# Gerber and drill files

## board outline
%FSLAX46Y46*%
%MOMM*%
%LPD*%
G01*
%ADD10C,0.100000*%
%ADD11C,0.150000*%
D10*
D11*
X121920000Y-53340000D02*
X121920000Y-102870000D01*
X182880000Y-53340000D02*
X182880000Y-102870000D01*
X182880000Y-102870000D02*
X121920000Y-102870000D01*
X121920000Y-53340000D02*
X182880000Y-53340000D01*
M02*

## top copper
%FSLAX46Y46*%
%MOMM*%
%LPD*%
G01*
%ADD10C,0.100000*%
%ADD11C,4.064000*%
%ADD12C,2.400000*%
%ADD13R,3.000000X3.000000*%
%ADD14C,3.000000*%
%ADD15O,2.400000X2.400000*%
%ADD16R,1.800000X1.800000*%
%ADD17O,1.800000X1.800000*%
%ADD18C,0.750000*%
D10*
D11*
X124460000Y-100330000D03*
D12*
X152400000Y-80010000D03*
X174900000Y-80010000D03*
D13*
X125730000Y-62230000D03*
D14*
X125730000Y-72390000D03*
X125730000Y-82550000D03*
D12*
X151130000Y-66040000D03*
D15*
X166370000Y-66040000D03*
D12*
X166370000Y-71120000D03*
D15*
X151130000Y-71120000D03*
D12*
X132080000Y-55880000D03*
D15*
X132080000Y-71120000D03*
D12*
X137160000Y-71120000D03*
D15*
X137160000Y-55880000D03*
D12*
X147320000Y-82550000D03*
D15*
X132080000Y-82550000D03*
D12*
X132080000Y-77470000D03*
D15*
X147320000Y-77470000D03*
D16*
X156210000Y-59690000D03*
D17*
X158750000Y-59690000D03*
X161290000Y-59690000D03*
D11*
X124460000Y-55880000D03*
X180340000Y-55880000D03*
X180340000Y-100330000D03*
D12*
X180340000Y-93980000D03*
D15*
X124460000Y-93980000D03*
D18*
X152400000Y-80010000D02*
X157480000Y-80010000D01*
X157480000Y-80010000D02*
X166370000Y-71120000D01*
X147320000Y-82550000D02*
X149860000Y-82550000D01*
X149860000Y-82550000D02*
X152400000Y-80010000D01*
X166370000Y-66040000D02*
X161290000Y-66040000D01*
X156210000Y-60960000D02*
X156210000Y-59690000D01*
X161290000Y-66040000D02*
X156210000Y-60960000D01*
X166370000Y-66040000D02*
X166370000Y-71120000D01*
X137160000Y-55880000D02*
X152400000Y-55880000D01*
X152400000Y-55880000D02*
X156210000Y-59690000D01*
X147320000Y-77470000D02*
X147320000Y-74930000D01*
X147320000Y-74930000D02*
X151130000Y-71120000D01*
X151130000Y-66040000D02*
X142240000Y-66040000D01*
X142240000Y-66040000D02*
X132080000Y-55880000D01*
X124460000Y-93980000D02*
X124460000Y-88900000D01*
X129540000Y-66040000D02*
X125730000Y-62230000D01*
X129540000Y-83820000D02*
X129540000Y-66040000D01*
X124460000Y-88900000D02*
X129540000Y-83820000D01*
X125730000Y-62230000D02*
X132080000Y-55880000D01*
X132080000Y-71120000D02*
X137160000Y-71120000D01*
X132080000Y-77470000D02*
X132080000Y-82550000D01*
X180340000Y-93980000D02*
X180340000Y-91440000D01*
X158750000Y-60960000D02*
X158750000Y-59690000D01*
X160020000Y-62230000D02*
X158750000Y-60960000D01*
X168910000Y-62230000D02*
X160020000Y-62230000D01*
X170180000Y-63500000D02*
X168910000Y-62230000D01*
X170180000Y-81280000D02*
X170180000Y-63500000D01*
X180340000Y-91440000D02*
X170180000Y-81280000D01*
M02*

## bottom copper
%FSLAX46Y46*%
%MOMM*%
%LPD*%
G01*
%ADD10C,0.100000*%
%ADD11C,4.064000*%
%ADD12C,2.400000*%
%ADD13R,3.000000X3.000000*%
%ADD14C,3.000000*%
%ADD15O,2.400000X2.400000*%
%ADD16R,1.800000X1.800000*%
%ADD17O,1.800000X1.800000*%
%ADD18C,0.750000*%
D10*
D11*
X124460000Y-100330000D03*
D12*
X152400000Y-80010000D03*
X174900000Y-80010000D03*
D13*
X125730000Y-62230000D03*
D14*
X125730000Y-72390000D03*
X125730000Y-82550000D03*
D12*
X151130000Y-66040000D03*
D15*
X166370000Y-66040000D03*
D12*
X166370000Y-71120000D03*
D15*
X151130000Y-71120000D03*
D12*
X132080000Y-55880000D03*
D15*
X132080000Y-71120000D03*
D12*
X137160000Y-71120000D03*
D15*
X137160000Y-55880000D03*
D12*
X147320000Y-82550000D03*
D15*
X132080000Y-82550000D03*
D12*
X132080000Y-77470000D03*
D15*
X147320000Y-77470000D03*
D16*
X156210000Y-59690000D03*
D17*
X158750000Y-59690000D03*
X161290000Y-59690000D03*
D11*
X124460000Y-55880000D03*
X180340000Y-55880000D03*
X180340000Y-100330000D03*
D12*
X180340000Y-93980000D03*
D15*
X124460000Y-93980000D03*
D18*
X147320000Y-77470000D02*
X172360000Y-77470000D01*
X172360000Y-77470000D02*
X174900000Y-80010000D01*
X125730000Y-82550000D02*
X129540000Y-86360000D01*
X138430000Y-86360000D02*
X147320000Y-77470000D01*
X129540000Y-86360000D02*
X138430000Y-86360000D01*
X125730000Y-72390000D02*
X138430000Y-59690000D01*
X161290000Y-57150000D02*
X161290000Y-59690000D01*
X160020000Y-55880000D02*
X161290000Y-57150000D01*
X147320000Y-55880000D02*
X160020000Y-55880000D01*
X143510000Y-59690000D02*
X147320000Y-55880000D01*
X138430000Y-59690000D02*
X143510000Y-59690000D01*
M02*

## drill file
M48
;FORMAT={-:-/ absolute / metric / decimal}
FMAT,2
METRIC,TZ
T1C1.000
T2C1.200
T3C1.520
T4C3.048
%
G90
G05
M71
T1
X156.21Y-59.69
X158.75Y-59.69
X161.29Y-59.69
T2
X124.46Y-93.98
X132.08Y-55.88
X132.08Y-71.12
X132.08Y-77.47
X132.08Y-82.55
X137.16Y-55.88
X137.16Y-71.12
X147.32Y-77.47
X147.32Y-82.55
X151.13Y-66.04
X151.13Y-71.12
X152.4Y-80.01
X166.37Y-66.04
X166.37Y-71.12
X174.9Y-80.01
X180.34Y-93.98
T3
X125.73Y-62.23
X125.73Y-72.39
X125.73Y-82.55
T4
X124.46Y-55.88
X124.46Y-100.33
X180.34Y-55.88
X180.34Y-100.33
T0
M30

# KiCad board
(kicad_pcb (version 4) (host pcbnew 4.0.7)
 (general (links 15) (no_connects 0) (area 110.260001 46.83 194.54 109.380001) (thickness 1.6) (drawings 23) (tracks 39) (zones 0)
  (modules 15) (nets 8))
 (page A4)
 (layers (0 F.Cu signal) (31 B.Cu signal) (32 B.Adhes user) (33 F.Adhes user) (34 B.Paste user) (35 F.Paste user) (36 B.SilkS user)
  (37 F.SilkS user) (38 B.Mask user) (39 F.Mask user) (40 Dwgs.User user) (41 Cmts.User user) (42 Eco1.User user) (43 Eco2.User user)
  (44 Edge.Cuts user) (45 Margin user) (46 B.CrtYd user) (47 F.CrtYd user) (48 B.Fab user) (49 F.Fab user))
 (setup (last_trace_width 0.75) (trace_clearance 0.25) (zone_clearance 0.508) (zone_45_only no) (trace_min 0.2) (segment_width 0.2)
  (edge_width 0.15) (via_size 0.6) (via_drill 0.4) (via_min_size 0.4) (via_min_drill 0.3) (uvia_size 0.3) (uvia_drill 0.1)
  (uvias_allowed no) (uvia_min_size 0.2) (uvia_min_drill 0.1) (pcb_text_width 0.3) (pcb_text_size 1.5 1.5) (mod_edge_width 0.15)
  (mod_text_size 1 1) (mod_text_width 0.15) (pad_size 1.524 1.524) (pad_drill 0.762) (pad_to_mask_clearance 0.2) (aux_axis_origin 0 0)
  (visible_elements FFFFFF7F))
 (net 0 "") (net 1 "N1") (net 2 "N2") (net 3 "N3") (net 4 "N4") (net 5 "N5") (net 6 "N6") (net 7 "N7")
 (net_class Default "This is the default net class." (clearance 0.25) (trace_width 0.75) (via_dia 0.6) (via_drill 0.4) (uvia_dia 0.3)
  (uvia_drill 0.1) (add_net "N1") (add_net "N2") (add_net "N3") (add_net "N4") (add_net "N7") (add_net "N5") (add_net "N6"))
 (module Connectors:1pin (layer F.Cu) (at 124.46 100.33)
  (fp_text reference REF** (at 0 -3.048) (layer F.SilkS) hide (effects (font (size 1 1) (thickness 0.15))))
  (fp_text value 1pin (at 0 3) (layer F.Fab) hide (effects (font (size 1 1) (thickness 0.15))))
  (pad 1 thru_hole circle (at 0 0) (size 4.064 4.064) (drill 3.048) (layers *.Cu *.Mask)))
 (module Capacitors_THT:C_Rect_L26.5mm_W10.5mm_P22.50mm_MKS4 (layer F.Cu) (at 152.4 80.01)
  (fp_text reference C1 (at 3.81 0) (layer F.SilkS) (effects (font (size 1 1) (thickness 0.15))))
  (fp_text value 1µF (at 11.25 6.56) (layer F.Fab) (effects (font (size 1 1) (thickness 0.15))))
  (pad 1 thru_hole circle (at 0 0) (size 2.4 2.4) (drill 1.2) (layers *.Cu *.Mask) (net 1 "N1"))
  (pad 2 thru_hole circle (at 22.5 0) (size 2.4 2.4) (drill 1.2) (layers *.Cu *.Mask) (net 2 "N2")))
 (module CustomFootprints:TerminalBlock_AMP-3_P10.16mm (layer F.Cu) (at 125.73 62.23 270)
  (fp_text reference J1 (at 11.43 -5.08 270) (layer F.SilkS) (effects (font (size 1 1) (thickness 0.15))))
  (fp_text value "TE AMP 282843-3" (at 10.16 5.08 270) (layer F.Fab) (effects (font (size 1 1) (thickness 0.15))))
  (pad 1 thru_hole rect (at 0 0 270) (size 3 3) (drill 1.52) (layers *.Cu *.Mask) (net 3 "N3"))
  (pad 2 thru_hole circle (at 10.16 0 270) (size 3 3) (drill 1.52) (layers *.Cu *.Mask) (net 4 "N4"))
  (pad 3 thru_hole circle (at 20.32 0 270) (size 3 3) (drill 1.52) (layers *.Cu *.Mask) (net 2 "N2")))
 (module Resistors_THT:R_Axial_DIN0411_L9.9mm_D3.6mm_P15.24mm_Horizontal (layer F.Cu) (at 151.13 66.04)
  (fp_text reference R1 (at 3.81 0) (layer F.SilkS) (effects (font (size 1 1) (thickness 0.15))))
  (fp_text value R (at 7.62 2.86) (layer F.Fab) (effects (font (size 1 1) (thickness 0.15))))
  (pad 1 thru_hole circle (at 0 0) (size 2.4 2.4) (drill 1.2) (layers *.Cu *.Mask) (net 3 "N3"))
  (pad 2 thru_hole oval (at 15.24 0) (size 2.4 2.4) (drill 1.2) (layers *.Cu *.Mask) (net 1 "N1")))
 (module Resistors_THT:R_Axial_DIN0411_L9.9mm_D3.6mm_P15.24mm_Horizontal (layer F.Cu) (at 166.37 71.12 180)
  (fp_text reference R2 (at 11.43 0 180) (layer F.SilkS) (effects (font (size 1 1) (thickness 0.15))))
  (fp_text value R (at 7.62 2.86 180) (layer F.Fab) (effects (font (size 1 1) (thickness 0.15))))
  (pad 1 thru_hole circle (at 0 0 180) (size 2.4 2.4) (drill 1.2) (layers *.Cu *.Mask) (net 1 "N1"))
  (pad 2 thru_hole oval (at 15.24 0 180) (size 2.4 2.4) (drill 1.2) (layers *.Cu *.Mask) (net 2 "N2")))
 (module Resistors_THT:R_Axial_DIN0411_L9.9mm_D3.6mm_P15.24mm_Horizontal (layer F.Cu) (at 132.08 55.88 270)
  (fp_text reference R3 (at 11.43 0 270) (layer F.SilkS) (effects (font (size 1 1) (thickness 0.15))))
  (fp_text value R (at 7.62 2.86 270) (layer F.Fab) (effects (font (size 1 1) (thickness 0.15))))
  (pad 1 thru_hole circle (at 0 0 270) (size 2.4 2.4) (drill 1.2) (layers *.Cu *.Mask) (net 3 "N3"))
  (pad 2 thru_hole oval (at 15.24 0 270) (size 2.4 2.4) (drill 1.2) (layers *.Cu *.Mask) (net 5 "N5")))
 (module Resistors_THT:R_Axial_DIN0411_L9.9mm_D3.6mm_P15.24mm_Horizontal (layer F.Cu) (at 137.16 71.12 90)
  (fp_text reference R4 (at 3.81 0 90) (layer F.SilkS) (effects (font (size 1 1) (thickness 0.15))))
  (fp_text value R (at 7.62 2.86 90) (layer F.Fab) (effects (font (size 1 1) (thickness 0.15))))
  (pad 1 thru_hole circle (at 0 0 90) (size 2.4 2.4) (drill 1.2) (layers *.Cu *.Mask) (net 5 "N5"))
  (pad 2 thru_hole oval (at 15.24 0 90) (size 2.4 2.4) (drill 1.2) (layers *.Cu *.Mask) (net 1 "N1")))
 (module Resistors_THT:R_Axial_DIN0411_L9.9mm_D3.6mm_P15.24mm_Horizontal (layer F.Cu) (at 147.32 82.55 180)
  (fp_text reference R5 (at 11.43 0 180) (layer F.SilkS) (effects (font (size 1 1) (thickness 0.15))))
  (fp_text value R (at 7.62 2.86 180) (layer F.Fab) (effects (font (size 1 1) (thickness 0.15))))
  (pad 1 thru_hole circle (at 0 0 180) (size 2.4 2.4) (drill 1.2) (layers *.Cu *.Mask) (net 1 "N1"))
  (pad 2 thru_hole oval (at 15.24 0 180) (size 2.4 2.4) (drill 1.2) (layers *.Cu *.Mask) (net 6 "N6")))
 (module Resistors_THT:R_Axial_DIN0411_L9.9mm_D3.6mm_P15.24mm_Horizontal (layer F.Cu) (at 132.08 77.47)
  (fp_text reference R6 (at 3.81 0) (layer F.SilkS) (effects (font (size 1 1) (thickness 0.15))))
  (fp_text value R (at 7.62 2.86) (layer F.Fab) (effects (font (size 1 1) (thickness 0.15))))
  (pad 1 thru_hole circle (at 0 0) (size 2.4 2.4) (drill 1.2) (layers *.Cu *.Mask) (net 6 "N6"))
  (pad 2 thru_hole oval (at 15.24 0) (size 2.4 2.4) (drill 1.2) (layers *.Cu *.Mask) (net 2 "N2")))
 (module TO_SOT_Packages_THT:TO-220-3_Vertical (layer F.Cu) (at 156.21 59.69)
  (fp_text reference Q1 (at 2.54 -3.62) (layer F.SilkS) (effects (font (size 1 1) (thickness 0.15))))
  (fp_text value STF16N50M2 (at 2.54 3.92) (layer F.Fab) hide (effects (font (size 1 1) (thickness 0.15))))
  (pad 1 thru_hole rect (at 0 0) (size 1.8 1.8) (drill 1) (layers *.Cu *.Mask) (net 1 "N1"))
  (pad 2 thru_hole oval (at 2.54 0) (size 1.8 1.8) (drill 1) (layers *.Cu *.Mask) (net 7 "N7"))
  (pad 3 thru_hole oval (at 5.08 0) (size 1.8 1.8) (drill 1) (layers *.Cu *.Mask) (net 4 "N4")))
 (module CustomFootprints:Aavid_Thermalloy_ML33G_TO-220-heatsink (layer F.Cu) (at 139.7 53.34)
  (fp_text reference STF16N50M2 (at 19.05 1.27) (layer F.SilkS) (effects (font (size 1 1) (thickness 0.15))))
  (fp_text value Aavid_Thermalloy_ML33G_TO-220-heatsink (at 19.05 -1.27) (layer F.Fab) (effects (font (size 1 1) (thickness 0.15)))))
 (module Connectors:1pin (layer F.Cu) (at 124.46 55.88)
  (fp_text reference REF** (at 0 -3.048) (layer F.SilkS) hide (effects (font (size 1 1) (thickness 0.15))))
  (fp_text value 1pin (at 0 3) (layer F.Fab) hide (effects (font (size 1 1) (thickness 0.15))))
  (pad 1 thru_hole circle (at 0 0) (size 4.064 4.064) (drill 3.048) (layers *.Cu *.Mask)))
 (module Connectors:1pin (layer F.Cu) (at 180.34 55.88)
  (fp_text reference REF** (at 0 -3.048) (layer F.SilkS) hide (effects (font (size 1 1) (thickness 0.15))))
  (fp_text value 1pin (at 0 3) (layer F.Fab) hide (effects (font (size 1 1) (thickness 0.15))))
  (pad 1 thru_hole circle (at 0 0) (size 4.064 4.064) (drill 3.048) (layers *.Cu *.Mask)))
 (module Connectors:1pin (layer F.Cu) (at 180.34 100.33)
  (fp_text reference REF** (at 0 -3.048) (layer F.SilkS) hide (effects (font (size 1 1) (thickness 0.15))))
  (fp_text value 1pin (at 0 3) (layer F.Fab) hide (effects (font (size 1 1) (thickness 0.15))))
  (pad 1 thru_hole circle (at 0 0) (size 4.064 4.064) (drill 3.048) (layers *.Cu *.Mask)))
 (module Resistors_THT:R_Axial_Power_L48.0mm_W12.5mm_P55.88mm (layer F.Cu) (at 180.34 93.98 180)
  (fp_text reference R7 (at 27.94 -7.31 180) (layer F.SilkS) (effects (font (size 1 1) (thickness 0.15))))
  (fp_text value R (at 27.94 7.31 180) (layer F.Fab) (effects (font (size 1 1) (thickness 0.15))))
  (pad 1 thru_hole circle (at 0 0 180) (size 2.4 2.4) (drill 1.2) (layers *.Cu *.Mask) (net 7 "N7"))
  (pad 2 thru_hole oval (at 55.88 0 180) (size 2.4 2.4) (drill 1.2) (layers *.Cu *.Mask) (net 3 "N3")))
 (gr_line (start 121.92 53.34) (end 121.92 102.87) (angle 90) (layer Edge.Cuts) (width 0.15))
 (gr_line (start 182.88 53.34) (end 182.88 102.87) (angle 90) (layer Edge.Cuts) (width 0.15))
 (gr_line (start 182.88 102.87) (end 121.92 102.87) (angle 90) (layer Edge.Cuts) (width 0.15))
 (gr_line (start 121.92 53.34) (end 182.88 53.34) (angle 90) (layer Edge.Cuts) (width 0.15))
 (segment (start 152.4 80.01) (end 157.48 80.01) (width 0.75) (layer F.Cu) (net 1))
 (segment (start 157.48 80.01) (end 166.37 71.12) (width 0.75) (layer F.Cu) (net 1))
 (segment (start 147.32 82.55) (end 149.86 82.55) (width 0.75) (layer F.Cu) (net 1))
 (segment (start 149.86 82.55) (end 152.4 80.01) (width 0.75) (layer F.Cu) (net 1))
 (segment (start 166.37 66.04) (end 161.29 66.04) (width 0.75) (layer F.Cu) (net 1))
 (segment (start 156.21 60.96) (end 156.21 59.69) (width 0.75) (layer F.Cu) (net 1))
 (segment (start 161.29 66.04) (end 156.21 60.96) (width 0.75) (layer F.Cu) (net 1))
 (segment (start 166.37 66.04) (end 166.37 71.12) (width 0.75) (layer F.Cu) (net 1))
 (segment (start 137.16 55.88) (end 152.4 55.88) (width 0.75) (layer F.Cu) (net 1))
 (segment (start 152.4 55.88) (end 156.21 59.69) (width 0.75) (layer F.Cu) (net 1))
 (segment (start 147.32 77.47) (end 172.36 77.47) (width 0.75) (layer B.Cu) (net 2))
 (segment (start 172.36 77.47) (end 174.9 80.01) (width 0.75) (layer B.Cu) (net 2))
 (segment (start 147.32 77.47) (end 147.32 74.93) (width 0.75) (layer F.Cu) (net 2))
 (segment (start 147.32 74.93) (end 151.13 71.12) (width 0.75) (layer F.Cu) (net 2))
 (segment (start 125.73 82.55) (end 129.54 86.36) (width 0.75) (layer B.Cu) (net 2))
 (segment (start 138.43 86.36) (end 147.32 77.47) (width 0.75) (layer B.Cu) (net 2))
 (segment (start 129.54 86.36) (end 138.43 86.36) (width 0.75) (layer B.Cu) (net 2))
 (segment (start 151.13 66.04) (end 142.24 66.04) (width 0.75) (layer F.Cu) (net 3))
 (segment (start 142.24 66.04) (end 132.08 55.88) (width 0.75) (layer F.Cu) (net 3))
 (segment (start 124.46 93.98) (end 124.46 88.9) (width 0.75) (layer F.Cu) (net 3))
 (segment (start 129.54 66.04) (end 125.73 62.23) (width 0.75) (layer F.Cu) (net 3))
 (segment (start 129.54 83.82) (end 129.54 66.04) (width 0.75) (layer F.Cu) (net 3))
 (segment (start 124.46 88.9) (end 129.54 83.82) (width 0.75) (layer F.Cu) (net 3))
 (segment (start 125.73 62.23) (end 132.08 55.88) (width 0.75) (layer F.Cu) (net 3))
 (segment (start 125.73 72.39) (end 138.43 59.69) (width 0.75) (layer B.Cu) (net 4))
 (segment (start 161.29 57.15) (end 161.29 59.69) (width 0.75) (layer B.Cu) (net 4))
 (segment (start 160.02 55.88) (end 161.29 57.15) (width 0.75) (layer B.Cu) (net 4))
 (segment (start 147.32 55.88) (end 160.02 55.88) (width 0.75) (layer B.Cu) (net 4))
 (segment (start 143.51 59.69) (end 147.32 55.88) (width 0.75) (layer B.Cu) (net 4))
 (segment (start 138.43 59.69) (end 143.51 59.69) (width 0.75) (layer B.Cu) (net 4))
 (segment (start 132.08 71.12) (end 137.16 71.12) (width 0.75) (layer F.Cu) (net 5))
 (segment (start 132.08 77.47) (end 132.08 82.55) (width 0.75) (layer F.Cu) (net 6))
 (segment (start 180.34 93.98) (end 180.34 91.44) (width 0.75) (layer F.Cu) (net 7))
 (segment (start 158.75 60.96) (end 158.75 59.69) (width 0.75) (layer F.Cu) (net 7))
 (segment (start 160.02 62.23) (end 158.75 60.96) (width 0.75) (layer F.Cu) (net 7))
 (segment (start 168.91 62.23) (end 160.02 62.23) (width 0.75) (layer F.Cu) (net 7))
 (segment (start 170.18 63.5) (end 168.91 62.23) (width 0.75) (layer F.Cu) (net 7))
 (segment (start 170.18 81.28) (end 170.18 63.5) (width 0.75) (layer F.Cu) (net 7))
 (segment (start 180.34 91.44) (end 170.18 81.28) (width 0.75) (layer F.Cu) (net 7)))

